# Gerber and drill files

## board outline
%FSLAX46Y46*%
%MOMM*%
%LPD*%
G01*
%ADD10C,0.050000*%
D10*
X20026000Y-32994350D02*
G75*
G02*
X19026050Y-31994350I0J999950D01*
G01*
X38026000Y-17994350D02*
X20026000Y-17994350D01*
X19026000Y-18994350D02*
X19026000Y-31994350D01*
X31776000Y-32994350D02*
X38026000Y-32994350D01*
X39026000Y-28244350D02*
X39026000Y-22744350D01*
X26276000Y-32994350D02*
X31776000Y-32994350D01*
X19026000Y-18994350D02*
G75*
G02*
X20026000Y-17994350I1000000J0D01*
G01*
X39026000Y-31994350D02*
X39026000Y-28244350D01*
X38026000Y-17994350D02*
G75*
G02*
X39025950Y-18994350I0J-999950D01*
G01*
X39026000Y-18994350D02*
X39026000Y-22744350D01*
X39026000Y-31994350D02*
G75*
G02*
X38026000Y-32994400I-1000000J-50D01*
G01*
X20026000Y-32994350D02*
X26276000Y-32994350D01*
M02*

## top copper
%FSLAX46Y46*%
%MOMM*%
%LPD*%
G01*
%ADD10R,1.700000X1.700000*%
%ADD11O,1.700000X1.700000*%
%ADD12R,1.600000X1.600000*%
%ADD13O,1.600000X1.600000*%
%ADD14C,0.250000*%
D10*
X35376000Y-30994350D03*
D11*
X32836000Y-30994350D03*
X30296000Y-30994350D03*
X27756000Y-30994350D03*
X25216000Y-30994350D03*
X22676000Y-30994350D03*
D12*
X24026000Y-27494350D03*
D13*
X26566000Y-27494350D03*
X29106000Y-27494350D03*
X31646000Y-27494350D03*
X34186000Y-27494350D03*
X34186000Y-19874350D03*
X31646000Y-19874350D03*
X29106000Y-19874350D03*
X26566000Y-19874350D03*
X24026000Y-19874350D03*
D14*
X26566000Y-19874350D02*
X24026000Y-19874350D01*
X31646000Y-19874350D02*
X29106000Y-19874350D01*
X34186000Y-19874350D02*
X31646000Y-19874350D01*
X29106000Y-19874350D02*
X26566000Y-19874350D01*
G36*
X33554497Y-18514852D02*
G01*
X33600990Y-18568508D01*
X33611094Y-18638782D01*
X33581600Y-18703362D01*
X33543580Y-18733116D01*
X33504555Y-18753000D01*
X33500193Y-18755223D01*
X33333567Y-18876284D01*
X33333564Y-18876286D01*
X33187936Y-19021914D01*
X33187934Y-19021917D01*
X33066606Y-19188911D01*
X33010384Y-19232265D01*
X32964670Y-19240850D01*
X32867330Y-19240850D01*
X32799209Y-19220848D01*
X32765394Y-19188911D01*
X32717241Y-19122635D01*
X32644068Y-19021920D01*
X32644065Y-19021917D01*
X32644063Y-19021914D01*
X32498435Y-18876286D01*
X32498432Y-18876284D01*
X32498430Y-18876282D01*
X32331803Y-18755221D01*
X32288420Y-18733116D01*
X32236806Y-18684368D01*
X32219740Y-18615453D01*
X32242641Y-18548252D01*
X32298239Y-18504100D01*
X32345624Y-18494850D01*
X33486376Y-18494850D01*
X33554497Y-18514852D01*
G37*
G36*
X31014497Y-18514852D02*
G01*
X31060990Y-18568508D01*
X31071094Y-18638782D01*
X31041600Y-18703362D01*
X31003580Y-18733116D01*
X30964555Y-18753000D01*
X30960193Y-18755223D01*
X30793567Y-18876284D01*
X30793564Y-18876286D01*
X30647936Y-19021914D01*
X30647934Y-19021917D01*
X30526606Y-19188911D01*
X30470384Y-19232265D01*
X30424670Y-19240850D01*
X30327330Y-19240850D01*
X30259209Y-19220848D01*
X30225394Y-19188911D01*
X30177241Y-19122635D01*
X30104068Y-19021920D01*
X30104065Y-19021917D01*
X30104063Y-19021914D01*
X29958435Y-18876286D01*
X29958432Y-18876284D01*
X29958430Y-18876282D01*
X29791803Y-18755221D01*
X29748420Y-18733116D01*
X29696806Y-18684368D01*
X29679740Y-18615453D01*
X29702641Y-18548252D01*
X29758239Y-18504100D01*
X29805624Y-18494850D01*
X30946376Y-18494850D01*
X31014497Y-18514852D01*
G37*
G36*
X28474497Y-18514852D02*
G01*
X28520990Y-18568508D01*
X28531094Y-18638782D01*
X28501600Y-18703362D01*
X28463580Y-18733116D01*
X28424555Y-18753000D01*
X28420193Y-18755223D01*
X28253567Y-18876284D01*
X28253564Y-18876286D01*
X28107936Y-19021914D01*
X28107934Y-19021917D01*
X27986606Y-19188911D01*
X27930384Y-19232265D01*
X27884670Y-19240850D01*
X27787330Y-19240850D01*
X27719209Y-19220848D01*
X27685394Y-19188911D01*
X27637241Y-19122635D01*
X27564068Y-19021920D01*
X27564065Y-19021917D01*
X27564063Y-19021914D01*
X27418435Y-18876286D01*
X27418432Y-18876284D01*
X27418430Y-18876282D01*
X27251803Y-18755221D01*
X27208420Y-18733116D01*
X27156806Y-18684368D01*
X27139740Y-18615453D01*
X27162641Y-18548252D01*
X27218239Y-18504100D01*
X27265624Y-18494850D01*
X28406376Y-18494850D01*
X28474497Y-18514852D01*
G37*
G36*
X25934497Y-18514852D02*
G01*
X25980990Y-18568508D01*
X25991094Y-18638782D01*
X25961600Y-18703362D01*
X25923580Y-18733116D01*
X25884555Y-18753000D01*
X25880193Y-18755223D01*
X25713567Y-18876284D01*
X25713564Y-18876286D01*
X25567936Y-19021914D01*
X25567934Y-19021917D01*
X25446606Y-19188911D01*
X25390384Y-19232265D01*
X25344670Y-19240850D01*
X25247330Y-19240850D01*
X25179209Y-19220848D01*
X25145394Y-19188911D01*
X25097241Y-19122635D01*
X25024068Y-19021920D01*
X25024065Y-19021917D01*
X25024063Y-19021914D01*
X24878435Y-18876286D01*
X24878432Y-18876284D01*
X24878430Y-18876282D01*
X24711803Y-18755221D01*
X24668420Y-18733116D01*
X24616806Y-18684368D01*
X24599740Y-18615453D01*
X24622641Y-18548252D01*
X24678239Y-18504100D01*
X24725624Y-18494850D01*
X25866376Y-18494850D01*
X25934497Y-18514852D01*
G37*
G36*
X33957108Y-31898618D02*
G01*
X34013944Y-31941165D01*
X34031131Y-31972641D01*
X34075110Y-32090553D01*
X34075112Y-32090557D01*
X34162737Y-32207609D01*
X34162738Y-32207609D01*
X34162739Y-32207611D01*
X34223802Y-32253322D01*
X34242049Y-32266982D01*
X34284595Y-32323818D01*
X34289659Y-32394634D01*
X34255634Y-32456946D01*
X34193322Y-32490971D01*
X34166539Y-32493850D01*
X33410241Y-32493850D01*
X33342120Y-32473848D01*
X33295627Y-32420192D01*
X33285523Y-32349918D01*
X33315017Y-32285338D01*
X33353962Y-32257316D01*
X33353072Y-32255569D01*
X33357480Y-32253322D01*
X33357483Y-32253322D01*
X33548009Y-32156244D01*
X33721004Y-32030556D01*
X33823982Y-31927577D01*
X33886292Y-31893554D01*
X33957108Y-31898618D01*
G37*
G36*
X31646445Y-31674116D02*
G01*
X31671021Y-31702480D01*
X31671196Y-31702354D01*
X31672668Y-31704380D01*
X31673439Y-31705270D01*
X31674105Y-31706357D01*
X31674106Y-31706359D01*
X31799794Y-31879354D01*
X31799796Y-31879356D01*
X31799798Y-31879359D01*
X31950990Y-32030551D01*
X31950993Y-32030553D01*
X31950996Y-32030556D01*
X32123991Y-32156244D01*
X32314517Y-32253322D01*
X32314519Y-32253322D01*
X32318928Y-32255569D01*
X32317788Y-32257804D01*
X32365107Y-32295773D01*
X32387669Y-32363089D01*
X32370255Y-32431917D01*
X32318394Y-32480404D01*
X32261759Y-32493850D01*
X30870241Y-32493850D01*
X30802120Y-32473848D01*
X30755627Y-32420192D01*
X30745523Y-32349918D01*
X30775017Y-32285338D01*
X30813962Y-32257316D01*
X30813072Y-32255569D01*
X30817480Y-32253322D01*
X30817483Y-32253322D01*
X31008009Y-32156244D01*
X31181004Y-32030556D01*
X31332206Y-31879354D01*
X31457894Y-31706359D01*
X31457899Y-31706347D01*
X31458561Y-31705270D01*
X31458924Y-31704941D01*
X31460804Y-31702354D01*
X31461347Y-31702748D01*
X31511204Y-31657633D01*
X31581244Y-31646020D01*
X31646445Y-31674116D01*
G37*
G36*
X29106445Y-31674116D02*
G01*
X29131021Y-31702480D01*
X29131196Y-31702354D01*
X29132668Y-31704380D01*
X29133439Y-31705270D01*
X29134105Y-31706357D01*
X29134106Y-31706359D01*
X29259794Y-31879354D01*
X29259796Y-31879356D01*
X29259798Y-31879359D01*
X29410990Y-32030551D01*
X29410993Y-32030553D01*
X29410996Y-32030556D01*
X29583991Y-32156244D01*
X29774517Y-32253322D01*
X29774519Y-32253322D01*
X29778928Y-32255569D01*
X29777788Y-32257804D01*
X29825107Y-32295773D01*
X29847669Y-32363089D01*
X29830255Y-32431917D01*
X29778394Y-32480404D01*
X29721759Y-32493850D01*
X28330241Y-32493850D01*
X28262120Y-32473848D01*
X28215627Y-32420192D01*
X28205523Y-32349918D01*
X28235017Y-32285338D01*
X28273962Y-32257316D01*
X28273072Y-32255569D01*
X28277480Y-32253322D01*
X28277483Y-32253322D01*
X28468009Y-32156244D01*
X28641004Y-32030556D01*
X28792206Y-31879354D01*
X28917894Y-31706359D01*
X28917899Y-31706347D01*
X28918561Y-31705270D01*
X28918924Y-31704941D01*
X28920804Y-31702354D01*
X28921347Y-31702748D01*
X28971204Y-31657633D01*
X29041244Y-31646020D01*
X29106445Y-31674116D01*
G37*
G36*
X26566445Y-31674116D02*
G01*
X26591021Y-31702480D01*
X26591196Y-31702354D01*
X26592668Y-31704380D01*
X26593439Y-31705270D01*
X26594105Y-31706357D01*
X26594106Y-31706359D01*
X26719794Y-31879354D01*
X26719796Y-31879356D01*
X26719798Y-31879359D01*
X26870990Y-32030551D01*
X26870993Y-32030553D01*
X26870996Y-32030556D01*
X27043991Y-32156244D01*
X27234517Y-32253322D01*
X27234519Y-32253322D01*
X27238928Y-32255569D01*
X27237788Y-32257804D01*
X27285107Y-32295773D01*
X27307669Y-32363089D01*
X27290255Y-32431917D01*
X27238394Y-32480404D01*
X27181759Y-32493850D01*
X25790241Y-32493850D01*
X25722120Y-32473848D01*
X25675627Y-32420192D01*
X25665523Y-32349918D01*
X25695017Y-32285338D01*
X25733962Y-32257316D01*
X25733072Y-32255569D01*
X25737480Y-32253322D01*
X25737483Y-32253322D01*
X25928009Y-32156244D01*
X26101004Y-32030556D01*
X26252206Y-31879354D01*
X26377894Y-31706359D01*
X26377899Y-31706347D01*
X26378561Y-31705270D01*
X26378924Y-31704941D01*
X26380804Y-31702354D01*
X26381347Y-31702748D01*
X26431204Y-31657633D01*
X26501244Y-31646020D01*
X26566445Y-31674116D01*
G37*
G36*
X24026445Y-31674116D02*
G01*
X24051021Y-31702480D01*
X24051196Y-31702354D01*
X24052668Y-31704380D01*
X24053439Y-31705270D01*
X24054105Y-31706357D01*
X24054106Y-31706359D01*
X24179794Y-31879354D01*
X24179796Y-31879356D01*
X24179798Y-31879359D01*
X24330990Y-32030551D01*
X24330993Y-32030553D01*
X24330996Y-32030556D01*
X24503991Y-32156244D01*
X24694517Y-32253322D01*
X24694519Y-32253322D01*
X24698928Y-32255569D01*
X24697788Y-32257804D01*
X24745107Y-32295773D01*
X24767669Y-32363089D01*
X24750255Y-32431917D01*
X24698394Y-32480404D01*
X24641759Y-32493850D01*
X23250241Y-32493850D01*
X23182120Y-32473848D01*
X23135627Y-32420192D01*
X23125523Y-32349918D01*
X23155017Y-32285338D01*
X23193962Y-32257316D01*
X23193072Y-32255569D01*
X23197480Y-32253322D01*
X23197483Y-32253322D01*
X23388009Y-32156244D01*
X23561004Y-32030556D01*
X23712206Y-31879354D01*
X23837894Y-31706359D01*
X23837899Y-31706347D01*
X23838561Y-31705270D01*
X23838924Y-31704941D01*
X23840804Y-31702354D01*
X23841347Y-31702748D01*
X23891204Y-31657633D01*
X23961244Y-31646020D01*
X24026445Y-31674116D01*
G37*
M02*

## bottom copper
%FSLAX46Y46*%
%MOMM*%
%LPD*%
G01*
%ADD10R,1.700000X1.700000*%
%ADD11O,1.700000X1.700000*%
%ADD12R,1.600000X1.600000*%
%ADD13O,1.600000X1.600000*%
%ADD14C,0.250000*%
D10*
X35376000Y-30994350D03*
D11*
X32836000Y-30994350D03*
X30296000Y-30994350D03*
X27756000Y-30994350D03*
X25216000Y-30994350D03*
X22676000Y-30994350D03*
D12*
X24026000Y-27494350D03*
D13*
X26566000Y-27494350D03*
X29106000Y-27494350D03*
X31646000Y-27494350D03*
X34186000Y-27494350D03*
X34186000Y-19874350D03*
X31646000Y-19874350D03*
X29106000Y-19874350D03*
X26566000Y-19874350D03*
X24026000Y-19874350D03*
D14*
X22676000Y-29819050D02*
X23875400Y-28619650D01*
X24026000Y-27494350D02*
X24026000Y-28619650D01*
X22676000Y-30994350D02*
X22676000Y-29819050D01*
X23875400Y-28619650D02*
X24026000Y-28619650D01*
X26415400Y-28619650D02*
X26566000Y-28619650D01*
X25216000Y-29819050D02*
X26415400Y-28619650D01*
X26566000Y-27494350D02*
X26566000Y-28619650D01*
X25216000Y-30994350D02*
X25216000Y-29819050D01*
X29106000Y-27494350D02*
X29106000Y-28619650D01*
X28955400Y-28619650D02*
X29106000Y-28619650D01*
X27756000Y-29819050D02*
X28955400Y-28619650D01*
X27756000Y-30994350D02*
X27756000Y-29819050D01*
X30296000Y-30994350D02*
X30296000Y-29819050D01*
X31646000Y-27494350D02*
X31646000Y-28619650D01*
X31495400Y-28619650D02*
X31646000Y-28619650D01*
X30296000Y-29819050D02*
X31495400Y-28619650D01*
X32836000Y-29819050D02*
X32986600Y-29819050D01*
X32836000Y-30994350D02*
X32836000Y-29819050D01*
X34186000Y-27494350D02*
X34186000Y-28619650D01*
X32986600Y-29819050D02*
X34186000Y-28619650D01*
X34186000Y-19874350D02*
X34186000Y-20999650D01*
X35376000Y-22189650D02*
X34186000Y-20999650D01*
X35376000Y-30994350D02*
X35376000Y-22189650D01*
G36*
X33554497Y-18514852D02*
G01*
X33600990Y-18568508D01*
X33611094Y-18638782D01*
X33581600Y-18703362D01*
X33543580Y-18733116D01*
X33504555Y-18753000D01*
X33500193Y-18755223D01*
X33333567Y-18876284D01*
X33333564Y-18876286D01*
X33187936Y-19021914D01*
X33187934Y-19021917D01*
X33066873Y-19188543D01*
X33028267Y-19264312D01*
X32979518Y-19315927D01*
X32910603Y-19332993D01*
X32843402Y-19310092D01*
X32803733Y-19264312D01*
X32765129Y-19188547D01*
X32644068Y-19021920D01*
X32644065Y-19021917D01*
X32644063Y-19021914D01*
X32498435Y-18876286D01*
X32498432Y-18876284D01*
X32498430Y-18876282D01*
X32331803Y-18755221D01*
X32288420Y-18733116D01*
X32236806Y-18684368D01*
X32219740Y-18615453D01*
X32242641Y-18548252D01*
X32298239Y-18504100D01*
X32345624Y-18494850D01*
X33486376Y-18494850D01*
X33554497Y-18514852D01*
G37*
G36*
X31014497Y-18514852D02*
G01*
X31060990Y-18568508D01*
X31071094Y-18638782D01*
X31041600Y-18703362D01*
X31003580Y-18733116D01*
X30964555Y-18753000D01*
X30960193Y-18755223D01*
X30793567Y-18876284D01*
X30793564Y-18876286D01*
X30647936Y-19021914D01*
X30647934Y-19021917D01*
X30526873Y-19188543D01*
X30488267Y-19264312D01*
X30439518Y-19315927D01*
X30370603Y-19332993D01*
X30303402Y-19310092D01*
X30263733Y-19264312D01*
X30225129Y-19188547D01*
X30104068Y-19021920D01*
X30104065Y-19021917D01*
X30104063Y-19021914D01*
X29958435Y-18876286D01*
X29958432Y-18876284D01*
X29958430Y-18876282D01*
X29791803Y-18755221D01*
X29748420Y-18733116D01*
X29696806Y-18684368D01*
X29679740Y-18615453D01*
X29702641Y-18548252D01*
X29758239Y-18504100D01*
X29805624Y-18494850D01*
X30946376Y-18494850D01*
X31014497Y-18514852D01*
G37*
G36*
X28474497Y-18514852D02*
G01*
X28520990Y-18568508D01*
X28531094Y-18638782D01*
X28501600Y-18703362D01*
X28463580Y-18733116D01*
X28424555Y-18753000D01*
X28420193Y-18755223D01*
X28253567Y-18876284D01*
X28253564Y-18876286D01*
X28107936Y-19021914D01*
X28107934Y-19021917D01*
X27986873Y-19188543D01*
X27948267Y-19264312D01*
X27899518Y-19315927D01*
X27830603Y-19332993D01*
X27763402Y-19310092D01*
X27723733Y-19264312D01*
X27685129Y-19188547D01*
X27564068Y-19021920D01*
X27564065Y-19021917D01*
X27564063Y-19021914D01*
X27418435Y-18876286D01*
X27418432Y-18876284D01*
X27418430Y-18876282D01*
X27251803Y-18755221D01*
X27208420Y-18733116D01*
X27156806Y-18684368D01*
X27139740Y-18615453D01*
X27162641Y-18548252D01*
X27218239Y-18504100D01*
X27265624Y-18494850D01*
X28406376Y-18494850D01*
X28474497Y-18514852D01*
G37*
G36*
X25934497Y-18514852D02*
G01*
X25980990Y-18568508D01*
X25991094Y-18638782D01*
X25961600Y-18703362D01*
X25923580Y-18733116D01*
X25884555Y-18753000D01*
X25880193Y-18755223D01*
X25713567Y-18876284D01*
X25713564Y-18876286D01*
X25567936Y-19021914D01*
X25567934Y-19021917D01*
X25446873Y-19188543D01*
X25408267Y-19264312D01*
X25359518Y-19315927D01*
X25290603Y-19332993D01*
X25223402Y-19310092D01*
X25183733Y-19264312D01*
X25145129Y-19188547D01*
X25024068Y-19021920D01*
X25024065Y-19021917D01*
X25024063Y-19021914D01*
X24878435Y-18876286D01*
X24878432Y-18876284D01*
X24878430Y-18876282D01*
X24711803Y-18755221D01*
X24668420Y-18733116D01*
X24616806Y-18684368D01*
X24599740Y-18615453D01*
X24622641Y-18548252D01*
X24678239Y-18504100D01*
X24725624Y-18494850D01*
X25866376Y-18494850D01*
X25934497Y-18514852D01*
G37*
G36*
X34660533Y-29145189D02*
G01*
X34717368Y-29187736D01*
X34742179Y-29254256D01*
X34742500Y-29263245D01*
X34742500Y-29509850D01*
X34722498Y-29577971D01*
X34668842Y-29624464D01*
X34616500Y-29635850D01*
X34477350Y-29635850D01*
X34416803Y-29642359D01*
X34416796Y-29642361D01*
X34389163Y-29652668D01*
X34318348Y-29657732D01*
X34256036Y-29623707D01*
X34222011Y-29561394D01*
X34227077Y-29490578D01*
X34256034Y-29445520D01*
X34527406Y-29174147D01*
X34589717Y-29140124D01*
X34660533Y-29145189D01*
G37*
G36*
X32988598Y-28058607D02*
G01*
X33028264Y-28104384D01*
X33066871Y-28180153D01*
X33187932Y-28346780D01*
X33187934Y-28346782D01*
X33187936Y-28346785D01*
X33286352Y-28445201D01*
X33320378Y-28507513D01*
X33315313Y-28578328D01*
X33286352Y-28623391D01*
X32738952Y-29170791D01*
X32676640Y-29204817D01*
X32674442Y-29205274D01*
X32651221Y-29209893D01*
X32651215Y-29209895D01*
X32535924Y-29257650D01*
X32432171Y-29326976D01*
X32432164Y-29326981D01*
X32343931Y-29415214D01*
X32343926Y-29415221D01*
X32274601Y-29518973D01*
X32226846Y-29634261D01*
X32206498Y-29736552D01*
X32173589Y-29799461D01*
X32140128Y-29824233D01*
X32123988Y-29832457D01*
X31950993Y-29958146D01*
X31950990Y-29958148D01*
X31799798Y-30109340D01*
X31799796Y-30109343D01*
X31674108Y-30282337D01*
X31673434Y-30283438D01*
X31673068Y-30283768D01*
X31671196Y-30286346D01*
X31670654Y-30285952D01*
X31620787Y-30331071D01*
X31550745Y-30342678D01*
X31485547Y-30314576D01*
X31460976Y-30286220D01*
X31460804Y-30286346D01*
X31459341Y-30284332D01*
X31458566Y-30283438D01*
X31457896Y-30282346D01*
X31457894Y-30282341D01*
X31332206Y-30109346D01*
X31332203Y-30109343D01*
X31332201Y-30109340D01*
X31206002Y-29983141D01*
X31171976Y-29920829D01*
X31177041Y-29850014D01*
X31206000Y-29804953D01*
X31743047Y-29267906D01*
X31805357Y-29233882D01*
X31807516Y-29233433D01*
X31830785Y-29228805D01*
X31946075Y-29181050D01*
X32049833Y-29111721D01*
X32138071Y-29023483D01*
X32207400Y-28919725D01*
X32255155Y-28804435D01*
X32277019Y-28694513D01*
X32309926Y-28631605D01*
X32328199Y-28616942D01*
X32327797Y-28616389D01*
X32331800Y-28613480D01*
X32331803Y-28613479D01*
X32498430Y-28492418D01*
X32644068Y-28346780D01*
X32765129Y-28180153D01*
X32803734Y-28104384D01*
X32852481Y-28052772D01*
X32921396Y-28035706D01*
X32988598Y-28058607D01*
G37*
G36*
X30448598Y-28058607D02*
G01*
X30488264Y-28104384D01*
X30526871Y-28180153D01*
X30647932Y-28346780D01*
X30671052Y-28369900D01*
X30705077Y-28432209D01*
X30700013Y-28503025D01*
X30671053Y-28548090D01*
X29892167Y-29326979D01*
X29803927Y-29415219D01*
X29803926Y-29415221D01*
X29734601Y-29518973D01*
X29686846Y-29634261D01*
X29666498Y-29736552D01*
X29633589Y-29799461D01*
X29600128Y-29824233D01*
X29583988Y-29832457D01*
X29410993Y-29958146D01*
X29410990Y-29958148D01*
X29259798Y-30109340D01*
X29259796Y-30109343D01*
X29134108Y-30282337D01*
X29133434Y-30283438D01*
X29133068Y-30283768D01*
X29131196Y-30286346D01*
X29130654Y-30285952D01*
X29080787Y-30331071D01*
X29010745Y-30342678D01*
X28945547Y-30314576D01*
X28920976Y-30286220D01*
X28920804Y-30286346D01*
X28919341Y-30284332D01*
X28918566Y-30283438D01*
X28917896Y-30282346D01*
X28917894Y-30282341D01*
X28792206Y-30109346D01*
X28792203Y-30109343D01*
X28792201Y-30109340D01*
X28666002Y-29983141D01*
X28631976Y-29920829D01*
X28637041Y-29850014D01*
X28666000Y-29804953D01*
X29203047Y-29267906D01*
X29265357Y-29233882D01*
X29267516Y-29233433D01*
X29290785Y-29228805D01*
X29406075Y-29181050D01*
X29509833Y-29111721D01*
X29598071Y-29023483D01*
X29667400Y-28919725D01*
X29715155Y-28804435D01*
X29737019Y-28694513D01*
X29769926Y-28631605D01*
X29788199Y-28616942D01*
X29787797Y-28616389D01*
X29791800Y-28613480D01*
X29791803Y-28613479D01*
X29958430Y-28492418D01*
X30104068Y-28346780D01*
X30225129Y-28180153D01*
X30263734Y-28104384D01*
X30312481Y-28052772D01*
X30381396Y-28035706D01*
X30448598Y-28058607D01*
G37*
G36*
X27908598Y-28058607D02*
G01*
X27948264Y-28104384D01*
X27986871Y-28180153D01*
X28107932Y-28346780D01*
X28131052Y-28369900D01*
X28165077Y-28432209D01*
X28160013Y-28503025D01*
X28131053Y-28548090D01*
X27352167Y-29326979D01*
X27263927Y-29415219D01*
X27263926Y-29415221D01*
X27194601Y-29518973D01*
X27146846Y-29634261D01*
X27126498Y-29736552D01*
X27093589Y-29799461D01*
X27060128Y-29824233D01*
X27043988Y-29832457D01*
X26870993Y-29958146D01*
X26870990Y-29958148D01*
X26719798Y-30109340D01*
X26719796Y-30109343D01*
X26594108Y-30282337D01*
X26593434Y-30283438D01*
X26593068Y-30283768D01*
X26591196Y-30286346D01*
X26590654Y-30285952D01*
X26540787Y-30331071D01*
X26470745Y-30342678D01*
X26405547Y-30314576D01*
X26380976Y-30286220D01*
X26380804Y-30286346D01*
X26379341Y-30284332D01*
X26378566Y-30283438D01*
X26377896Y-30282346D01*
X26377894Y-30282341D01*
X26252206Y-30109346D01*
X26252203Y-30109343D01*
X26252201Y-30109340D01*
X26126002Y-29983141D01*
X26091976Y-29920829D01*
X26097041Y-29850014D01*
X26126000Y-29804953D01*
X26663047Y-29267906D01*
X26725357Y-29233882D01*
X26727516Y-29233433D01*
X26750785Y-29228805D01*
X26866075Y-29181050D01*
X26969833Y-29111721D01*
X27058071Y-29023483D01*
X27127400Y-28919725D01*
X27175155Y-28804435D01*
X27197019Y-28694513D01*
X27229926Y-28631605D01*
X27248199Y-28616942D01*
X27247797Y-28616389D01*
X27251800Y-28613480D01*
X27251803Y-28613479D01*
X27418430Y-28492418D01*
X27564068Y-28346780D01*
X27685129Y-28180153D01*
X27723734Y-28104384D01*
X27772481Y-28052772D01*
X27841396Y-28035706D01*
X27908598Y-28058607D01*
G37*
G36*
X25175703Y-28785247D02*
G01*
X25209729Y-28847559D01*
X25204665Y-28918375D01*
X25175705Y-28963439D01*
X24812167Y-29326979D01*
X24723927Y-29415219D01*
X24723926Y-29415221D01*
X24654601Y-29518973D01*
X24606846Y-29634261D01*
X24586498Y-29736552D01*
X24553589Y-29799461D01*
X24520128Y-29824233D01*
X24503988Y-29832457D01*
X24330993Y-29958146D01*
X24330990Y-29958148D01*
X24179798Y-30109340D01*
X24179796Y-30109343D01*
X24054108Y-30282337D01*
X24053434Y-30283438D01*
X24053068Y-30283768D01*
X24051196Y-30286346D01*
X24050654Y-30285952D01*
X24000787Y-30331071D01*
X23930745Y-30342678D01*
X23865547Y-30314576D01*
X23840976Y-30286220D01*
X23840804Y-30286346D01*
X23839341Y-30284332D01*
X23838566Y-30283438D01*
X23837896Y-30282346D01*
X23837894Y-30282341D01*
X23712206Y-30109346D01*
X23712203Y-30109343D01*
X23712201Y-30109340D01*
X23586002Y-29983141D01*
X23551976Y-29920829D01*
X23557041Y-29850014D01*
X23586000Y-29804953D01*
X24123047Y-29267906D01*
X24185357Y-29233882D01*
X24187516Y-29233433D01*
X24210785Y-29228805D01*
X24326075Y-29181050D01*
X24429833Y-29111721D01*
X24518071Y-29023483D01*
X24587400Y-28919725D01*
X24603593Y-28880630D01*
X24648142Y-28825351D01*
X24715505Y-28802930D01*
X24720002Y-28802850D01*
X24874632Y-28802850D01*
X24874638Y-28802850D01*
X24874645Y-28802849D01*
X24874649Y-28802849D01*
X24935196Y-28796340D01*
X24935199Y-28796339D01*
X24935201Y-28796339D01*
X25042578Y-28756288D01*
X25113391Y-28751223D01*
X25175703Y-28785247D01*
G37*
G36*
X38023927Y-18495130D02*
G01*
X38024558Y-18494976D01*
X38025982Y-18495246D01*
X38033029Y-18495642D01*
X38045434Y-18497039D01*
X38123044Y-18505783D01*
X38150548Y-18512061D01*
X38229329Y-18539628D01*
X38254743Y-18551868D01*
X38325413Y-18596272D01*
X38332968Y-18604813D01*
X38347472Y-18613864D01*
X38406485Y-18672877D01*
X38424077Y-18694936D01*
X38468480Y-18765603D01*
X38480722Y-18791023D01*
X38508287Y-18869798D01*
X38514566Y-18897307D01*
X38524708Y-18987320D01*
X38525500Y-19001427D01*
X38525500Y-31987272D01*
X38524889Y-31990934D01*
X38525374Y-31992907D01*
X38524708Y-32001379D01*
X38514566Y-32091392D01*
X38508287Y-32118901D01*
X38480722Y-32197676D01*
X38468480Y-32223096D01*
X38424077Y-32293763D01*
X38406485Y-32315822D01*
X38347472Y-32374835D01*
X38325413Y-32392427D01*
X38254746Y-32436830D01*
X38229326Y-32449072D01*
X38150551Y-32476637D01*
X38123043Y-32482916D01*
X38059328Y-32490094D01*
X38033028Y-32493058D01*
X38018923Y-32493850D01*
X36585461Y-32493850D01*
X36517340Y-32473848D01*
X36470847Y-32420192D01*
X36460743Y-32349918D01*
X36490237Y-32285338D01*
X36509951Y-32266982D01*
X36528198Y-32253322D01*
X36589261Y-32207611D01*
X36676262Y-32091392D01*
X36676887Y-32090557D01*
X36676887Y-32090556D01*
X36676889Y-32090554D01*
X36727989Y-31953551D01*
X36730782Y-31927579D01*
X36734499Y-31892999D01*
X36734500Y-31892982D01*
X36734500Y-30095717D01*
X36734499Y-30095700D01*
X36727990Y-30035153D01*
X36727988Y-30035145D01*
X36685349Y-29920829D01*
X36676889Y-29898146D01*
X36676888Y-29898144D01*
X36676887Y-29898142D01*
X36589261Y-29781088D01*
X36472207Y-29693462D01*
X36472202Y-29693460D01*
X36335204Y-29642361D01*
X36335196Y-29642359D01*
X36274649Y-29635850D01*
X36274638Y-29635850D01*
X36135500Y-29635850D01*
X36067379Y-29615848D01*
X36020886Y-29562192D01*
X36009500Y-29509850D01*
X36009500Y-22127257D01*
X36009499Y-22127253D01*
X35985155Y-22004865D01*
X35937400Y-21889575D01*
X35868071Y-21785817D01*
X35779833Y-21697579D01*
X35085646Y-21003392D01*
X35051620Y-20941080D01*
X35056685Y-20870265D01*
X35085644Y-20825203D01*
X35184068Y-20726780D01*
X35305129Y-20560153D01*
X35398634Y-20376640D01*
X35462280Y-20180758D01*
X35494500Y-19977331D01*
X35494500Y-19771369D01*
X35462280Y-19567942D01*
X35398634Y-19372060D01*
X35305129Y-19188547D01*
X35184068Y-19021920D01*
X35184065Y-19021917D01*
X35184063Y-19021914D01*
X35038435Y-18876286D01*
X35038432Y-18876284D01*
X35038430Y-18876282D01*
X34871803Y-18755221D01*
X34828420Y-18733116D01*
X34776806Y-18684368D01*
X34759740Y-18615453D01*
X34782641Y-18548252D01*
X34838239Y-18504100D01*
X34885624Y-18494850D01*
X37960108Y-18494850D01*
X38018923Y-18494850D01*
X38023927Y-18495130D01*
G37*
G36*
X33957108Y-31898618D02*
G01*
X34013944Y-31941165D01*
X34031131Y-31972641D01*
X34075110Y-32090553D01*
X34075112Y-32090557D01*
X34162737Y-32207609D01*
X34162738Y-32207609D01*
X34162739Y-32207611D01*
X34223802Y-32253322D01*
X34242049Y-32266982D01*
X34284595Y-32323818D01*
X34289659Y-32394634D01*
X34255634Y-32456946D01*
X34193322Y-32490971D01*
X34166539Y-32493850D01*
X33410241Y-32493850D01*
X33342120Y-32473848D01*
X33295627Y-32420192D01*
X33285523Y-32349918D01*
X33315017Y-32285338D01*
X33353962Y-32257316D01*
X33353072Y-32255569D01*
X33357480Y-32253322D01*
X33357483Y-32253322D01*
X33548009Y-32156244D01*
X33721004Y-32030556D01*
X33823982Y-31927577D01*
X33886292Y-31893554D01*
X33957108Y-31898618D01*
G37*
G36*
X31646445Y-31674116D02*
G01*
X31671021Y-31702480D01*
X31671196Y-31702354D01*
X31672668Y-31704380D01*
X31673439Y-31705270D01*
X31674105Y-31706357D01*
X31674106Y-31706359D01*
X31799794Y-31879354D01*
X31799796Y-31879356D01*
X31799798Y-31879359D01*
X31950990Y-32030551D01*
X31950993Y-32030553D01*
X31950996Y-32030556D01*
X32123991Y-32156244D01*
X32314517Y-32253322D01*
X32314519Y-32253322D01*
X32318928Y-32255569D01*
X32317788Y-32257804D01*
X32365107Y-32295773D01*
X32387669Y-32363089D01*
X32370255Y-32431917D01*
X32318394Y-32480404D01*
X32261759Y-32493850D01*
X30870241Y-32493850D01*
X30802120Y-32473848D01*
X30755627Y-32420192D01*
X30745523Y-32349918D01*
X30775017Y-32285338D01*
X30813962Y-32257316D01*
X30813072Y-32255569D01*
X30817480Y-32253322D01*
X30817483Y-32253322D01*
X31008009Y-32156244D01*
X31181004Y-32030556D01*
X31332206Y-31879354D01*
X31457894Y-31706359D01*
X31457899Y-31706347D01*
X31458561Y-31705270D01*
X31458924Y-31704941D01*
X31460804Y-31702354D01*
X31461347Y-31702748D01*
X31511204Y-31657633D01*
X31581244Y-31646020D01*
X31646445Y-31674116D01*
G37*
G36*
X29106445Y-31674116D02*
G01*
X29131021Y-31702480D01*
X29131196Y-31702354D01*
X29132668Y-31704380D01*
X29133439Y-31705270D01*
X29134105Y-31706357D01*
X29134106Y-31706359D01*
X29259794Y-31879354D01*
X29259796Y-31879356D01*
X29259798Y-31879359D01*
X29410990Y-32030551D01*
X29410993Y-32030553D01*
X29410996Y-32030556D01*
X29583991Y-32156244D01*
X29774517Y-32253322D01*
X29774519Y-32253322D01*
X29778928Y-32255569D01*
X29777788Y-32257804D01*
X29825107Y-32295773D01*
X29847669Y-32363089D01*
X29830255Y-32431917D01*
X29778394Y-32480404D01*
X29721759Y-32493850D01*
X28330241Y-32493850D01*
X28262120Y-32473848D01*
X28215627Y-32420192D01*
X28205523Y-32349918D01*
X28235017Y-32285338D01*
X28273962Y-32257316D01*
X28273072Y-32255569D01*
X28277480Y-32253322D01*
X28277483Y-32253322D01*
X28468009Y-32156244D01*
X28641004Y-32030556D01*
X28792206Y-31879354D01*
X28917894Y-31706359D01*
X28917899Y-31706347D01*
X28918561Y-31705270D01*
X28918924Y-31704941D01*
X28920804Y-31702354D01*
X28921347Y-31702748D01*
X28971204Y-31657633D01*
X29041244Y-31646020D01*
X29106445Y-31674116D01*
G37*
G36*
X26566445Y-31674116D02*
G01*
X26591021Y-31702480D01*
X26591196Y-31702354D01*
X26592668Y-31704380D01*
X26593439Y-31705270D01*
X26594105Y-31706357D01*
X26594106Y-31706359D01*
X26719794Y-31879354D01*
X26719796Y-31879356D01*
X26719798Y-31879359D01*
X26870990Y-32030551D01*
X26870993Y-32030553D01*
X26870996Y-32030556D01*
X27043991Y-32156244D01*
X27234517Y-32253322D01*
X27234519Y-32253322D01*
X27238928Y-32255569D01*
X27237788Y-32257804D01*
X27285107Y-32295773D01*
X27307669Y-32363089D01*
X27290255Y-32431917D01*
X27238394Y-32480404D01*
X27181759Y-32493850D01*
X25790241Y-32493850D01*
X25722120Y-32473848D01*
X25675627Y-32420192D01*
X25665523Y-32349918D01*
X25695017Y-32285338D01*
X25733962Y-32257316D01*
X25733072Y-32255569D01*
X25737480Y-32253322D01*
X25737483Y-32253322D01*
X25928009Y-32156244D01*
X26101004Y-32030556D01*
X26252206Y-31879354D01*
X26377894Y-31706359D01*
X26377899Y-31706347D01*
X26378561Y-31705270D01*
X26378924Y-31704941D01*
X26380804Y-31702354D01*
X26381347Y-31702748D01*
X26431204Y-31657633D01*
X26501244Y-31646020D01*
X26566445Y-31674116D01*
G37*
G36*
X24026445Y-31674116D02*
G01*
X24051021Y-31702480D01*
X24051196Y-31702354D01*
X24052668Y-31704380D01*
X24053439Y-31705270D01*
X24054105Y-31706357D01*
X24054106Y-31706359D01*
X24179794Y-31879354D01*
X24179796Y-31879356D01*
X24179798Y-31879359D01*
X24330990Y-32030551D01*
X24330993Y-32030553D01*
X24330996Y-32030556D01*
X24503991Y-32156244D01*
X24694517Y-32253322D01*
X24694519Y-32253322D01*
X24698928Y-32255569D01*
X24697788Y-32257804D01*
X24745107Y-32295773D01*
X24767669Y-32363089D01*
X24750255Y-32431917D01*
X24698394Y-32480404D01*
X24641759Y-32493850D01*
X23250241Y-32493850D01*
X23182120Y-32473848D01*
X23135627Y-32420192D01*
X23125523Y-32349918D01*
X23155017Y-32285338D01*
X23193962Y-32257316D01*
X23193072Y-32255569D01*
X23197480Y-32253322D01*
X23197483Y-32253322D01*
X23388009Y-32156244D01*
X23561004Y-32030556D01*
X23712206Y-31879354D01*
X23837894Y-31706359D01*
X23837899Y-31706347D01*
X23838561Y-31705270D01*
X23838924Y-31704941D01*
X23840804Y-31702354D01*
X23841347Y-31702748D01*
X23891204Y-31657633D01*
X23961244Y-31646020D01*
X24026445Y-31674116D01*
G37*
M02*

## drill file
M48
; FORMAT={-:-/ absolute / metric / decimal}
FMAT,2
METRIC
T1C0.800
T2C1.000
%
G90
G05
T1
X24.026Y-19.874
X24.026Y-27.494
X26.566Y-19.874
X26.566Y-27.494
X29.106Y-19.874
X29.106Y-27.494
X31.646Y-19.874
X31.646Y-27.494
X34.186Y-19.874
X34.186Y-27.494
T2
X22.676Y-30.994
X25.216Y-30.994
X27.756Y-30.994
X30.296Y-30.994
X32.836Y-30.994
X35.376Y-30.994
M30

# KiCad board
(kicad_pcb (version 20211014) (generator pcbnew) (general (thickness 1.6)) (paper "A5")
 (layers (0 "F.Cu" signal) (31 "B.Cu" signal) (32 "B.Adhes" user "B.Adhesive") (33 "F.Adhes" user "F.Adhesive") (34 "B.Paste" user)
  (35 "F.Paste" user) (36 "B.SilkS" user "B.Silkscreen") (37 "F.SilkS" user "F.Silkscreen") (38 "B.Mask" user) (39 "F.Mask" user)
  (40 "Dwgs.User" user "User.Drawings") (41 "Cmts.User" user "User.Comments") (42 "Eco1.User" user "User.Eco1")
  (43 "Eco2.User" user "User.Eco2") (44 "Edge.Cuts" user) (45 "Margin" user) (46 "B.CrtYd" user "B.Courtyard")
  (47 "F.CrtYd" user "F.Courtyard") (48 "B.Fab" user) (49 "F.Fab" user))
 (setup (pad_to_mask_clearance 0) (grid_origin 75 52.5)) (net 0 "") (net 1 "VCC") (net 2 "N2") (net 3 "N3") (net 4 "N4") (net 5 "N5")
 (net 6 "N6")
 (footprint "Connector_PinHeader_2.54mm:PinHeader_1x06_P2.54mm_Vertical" (layer "F.Cu") (at 35.376 30.99435 -90)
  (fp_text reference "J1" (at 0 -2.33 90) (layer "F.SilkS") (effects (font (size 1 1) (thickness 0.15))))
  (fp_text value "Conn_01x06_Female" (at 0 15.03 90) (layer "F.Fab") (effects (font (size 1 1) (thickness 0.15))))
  (pad "1" thru_hole rect locked (at 0 0 270) (size 1.7 1.7) (drill 1) (layers *.Cu *.Mask) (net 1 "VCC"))
  (pad "2" thru_hole oval locked (at 0 2.54 270) (size 1.7 1.7) (drill 1) (layers *.Cu *.Mask) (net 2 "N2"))
  (pad "3" thru_hole oval locked (at 0 5.08 270) (size 1.7 1.7) (drill 1) (layers *.Cu *.Mask) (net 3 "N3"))
  (pad "4" thru_hole oval locked (at 0 7.62 270) (size 1.7 1.7) (drill 1) (layers *.Cu *.Mask) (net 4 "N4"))
  (pad "5" thru_hole oval locked (at 0 10.16 270) (size 1.7 1.7) (drill 1) (layers *.Cu *.Mask) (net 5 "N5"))
  (pad "6" thru_hole oval locked (at 0 12.7 270) (size 1.7 1.7) (drill 1) (layers *.Cu *.Mask) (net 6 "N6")))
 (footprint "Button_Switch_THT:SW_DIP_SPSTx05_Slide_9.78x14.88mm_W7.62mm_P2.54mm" (layer "F.Cu") (at 24.026 27.49435 90)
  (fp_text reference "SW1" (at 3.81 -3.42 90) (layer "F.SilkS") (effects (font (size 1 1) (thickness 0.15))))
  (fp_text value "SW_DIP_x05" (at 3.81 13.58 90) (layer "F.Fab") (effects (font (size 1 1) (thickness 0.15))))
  (pad "1" thru_hole rect locked (at 0 0 90) (size 1.6 1.6) (drill 0.8) (layers *.Cu *.Mask) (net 6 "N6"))
  (pad "2" thru_hole oval locked (at 0 2.54 90) (size 1.6 1.6) (drill 0.8) (layers *.Cu *.Mask) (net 5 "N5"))
  (pad "3" thru_hole oval locked (at 0 5.08 90) (size 1.6 1.6) (drill 0.8) (layers *.Cu *.Mask) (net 4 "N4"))
  (pad "4" thru_hole oval locked (at 0 7.62 90) (size 1.6 1.6) (drill 0.8) (layers *.Cu *.Mask) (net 3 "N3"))
  (pad "5" thru_hole oval locked (at 0 10.16 90) (size 1.6 1.6) (drill 0.8) (layers *.Cu *.Mask) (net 2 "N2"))
  (pad "6" thru_hole oval locked (at 7.62 10.16 90) (size 1.6 1.6) (drill 0.8) (layers *.Cu *.Mask) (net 1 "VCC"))
  (pad "7" thru_hole oval locked (at 7.62 7.62 90) (size 1.6 1.6) (drill 0.8) (layers *.Cu *.Mask) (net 1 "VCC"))
  (pad "8" thru_hole oval locked (at 7.62 5.08 90) (size 1.6 1.6) (drill 0.8) (layers *.Cu *.Mask) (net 1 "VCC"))
  (pad "9" thru_hole oval locked (at 7.62 2.54 90) (size 1.6 1.6) (drill 0.8) (layers *.Cu *.Mask) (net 1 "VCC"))
  (pad "10" thru_hole oval locked (at 7.62 0 90) (size 1.6 1.6) (drill 0.8) (layers *.Cu *.Mask) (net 1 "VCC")))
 (gr_arc (start 20.026 32.99435) (mid 19.318893 32.701457) (end 19.026 31.99435) (layer "Edge.Cuts") (width 0.05))
 (gr_line (start 38.026 17.99435) (end 20.026 17.99435) (layer "Edge.Cuts") (width 0.05))
 (gr_line (start 19.026 18.99435) (end 19.026 31.99435) (layer "Edge.Cuts") (width 0.05))
 (gr_line (start 31.776 32.99435) (end 38.026 32.99435) (layer "Edge.Cuts") (width 0.05))
 (gr_line (start 39.026 28.24435) (end 39.026 22.74435) (layer "Edge.Cuts") (width 0.05))
 (gr_line (start 26.276 32.99435) (end 31.776 32.99435) (layer "Edge.Cuts") (width 0.05))
 (gr_arc (start 19.026 18.99435) (mid 19.318893 18.287243) (end 20.026 17.99435) (layer "Edge.Cuts") (width 0.05))
 (gr_line (start 39.026 31.99435) (end 39.026 28.24435) (layer "Edge.Cuts") (width 0.05))
 (gr_arc (start 38.026 17.99435) (mid 38.733107 18.287243) (end 39.026 18.99435) (layer "Edge.Cuts") (width 0.05))
 (gr_line (start 39.026 18.99435) (end 39.026 22.74435) (layer "Edge.Cuts") (width 0.05))
 (gr_arc (start 39.026 31.99435) (mid 38.733107 32.701457) (end 38.026 32.99435) (layer "Edge.Cuts") (width 0.05))
 (gr_line (start 20.026 32.99435) (end 26.276 32.99435) (layer "Edge.Cuts") (width 0.05))
 (segment (start 22.676 29.81905) (end 23.8754 28.61965) (width 0.25) (layer "B.Cu") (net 6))
 (segment (start 24.026 27.49435) (end 24.026 28.61965) (width 0.25) (layer "B.Cu") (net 6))
 (segment (start 22.676 30.99435) (end 22.676 29.81905) (width 0.25) (layer "B.Cu") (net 6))
 (segment (start 23.8754 28.61965) (end 24.026 28.61965) (width 0.25) (layer "B.Cu") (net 6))
 (segment (start 26.4154 28.61965) (end 26.566 28.61965) (width 0.25) (layer "B.Cu") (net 5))
 (segment (start 25.216 29.81905) (end 26.4154 28.61965) (width 0.25) (layer "B.Cu") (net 5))
 (segment (start 26.566 27.49435) (end 26.566 28.61965) (width 0.25) (layer "B.Cu") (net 5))
 (segment (start 25.216 30.99435) (end 25.216 29.81905) (width 0.25) (layer "B.Cu") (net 5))
 (segment (start 29.106 27.49435) (end 29.106 28.61965) (width 0.25) (layer "B.Cu") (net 4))
 (segment (start 28.9554 28.61965) (end 29.106 28.61965) (width 0.25) (layer "B.Cu") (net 4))
 (segment (start 27.756 29.81905) (end 28.9554 28.61965) (width 0.25) (layer "B.Cu") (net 4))
 (segment (start 27.756 30.99435) (end 27.756 29.81905) (width 0.25) (layer "B.Cu") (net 4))
 (segment (start 30.296 30.99435) (end 30.296 29.81905) (width 0.25) (layer "B.Cu") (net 3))
 (segment (start 31.646 27.49435) (end 31.646 28.61965) (width 0.25) (layer "B.Cu") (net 3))
 (segment (start 31.4954 28.61965) (end 31.646 28.61965) (width 0.25) (layer "B.Cu") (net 3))
 (segment (start 30.296 29.81905) (end 31.4954 28.61965) (width 0.25) (layer "B.Cu") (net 3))
 (segment (start 32.836 29.81905) (end 32.9866 29.81905) (width 0.25) (layer "B.Cu") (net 2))
 (segment (start 32.836 30.99435) (end 32.836 29.81905) (width 0.25) (layer "B.Cu") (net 2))
 (segment (start 34.186 27.49435) (end 34.186 28.61965) (width 0.25) (layer "B.Cu") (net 2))
 (segment (start 32.9866 29.81905) (end 34.186 28.61965) (width 0.25) (layer "B.Cu") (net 2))
 (segment (start 26.566 19.87435) (end 24.026 19.87435) (width 0.25) (layer "F.Cu") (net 1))
 (segment (start 31.646 19.87435) (end 29.106 19.87435) (width 0.25) (layer "F.Cu") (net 1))
 (segment (start 34.186 19.87435) (end 31.646 19.87435) (width 0.25) (layer "F.Cu") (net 1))
 (segment (start 29.106 19.87435) (end 26.566 19.87435) (width 0.25) (layer "F.Cu") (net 1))
 (segment (start 34.186 19.87435) (end 34.186 20.99965) (width 0.25) (layer "B.Cu") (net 1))
 (segment (start 35.376 22.18965) (end 34.186 20.99965) (width 0.25) (layer "B.Cu") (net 1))
 (segment (start 35.376 30.99435) (end 35.376 22.18965) (width 0.25) (layer "B.Cu") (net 1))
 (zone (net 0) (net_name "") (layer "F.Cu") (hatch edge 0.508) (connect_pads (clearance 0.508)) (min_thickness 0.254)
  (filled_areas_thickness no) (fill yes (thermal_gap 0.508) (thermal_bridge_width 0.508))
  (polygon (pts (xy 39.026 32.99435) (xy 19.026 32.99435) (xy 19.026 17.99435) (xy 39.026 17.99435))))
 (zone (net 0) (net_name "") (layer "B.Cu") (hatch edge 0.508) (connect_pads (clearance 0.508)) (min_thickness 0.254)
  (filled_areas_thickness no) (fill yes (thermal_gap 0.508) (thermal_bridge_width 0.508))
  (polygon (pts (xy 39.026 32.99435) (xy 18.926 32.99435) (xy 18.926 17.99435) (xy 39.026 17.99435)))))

